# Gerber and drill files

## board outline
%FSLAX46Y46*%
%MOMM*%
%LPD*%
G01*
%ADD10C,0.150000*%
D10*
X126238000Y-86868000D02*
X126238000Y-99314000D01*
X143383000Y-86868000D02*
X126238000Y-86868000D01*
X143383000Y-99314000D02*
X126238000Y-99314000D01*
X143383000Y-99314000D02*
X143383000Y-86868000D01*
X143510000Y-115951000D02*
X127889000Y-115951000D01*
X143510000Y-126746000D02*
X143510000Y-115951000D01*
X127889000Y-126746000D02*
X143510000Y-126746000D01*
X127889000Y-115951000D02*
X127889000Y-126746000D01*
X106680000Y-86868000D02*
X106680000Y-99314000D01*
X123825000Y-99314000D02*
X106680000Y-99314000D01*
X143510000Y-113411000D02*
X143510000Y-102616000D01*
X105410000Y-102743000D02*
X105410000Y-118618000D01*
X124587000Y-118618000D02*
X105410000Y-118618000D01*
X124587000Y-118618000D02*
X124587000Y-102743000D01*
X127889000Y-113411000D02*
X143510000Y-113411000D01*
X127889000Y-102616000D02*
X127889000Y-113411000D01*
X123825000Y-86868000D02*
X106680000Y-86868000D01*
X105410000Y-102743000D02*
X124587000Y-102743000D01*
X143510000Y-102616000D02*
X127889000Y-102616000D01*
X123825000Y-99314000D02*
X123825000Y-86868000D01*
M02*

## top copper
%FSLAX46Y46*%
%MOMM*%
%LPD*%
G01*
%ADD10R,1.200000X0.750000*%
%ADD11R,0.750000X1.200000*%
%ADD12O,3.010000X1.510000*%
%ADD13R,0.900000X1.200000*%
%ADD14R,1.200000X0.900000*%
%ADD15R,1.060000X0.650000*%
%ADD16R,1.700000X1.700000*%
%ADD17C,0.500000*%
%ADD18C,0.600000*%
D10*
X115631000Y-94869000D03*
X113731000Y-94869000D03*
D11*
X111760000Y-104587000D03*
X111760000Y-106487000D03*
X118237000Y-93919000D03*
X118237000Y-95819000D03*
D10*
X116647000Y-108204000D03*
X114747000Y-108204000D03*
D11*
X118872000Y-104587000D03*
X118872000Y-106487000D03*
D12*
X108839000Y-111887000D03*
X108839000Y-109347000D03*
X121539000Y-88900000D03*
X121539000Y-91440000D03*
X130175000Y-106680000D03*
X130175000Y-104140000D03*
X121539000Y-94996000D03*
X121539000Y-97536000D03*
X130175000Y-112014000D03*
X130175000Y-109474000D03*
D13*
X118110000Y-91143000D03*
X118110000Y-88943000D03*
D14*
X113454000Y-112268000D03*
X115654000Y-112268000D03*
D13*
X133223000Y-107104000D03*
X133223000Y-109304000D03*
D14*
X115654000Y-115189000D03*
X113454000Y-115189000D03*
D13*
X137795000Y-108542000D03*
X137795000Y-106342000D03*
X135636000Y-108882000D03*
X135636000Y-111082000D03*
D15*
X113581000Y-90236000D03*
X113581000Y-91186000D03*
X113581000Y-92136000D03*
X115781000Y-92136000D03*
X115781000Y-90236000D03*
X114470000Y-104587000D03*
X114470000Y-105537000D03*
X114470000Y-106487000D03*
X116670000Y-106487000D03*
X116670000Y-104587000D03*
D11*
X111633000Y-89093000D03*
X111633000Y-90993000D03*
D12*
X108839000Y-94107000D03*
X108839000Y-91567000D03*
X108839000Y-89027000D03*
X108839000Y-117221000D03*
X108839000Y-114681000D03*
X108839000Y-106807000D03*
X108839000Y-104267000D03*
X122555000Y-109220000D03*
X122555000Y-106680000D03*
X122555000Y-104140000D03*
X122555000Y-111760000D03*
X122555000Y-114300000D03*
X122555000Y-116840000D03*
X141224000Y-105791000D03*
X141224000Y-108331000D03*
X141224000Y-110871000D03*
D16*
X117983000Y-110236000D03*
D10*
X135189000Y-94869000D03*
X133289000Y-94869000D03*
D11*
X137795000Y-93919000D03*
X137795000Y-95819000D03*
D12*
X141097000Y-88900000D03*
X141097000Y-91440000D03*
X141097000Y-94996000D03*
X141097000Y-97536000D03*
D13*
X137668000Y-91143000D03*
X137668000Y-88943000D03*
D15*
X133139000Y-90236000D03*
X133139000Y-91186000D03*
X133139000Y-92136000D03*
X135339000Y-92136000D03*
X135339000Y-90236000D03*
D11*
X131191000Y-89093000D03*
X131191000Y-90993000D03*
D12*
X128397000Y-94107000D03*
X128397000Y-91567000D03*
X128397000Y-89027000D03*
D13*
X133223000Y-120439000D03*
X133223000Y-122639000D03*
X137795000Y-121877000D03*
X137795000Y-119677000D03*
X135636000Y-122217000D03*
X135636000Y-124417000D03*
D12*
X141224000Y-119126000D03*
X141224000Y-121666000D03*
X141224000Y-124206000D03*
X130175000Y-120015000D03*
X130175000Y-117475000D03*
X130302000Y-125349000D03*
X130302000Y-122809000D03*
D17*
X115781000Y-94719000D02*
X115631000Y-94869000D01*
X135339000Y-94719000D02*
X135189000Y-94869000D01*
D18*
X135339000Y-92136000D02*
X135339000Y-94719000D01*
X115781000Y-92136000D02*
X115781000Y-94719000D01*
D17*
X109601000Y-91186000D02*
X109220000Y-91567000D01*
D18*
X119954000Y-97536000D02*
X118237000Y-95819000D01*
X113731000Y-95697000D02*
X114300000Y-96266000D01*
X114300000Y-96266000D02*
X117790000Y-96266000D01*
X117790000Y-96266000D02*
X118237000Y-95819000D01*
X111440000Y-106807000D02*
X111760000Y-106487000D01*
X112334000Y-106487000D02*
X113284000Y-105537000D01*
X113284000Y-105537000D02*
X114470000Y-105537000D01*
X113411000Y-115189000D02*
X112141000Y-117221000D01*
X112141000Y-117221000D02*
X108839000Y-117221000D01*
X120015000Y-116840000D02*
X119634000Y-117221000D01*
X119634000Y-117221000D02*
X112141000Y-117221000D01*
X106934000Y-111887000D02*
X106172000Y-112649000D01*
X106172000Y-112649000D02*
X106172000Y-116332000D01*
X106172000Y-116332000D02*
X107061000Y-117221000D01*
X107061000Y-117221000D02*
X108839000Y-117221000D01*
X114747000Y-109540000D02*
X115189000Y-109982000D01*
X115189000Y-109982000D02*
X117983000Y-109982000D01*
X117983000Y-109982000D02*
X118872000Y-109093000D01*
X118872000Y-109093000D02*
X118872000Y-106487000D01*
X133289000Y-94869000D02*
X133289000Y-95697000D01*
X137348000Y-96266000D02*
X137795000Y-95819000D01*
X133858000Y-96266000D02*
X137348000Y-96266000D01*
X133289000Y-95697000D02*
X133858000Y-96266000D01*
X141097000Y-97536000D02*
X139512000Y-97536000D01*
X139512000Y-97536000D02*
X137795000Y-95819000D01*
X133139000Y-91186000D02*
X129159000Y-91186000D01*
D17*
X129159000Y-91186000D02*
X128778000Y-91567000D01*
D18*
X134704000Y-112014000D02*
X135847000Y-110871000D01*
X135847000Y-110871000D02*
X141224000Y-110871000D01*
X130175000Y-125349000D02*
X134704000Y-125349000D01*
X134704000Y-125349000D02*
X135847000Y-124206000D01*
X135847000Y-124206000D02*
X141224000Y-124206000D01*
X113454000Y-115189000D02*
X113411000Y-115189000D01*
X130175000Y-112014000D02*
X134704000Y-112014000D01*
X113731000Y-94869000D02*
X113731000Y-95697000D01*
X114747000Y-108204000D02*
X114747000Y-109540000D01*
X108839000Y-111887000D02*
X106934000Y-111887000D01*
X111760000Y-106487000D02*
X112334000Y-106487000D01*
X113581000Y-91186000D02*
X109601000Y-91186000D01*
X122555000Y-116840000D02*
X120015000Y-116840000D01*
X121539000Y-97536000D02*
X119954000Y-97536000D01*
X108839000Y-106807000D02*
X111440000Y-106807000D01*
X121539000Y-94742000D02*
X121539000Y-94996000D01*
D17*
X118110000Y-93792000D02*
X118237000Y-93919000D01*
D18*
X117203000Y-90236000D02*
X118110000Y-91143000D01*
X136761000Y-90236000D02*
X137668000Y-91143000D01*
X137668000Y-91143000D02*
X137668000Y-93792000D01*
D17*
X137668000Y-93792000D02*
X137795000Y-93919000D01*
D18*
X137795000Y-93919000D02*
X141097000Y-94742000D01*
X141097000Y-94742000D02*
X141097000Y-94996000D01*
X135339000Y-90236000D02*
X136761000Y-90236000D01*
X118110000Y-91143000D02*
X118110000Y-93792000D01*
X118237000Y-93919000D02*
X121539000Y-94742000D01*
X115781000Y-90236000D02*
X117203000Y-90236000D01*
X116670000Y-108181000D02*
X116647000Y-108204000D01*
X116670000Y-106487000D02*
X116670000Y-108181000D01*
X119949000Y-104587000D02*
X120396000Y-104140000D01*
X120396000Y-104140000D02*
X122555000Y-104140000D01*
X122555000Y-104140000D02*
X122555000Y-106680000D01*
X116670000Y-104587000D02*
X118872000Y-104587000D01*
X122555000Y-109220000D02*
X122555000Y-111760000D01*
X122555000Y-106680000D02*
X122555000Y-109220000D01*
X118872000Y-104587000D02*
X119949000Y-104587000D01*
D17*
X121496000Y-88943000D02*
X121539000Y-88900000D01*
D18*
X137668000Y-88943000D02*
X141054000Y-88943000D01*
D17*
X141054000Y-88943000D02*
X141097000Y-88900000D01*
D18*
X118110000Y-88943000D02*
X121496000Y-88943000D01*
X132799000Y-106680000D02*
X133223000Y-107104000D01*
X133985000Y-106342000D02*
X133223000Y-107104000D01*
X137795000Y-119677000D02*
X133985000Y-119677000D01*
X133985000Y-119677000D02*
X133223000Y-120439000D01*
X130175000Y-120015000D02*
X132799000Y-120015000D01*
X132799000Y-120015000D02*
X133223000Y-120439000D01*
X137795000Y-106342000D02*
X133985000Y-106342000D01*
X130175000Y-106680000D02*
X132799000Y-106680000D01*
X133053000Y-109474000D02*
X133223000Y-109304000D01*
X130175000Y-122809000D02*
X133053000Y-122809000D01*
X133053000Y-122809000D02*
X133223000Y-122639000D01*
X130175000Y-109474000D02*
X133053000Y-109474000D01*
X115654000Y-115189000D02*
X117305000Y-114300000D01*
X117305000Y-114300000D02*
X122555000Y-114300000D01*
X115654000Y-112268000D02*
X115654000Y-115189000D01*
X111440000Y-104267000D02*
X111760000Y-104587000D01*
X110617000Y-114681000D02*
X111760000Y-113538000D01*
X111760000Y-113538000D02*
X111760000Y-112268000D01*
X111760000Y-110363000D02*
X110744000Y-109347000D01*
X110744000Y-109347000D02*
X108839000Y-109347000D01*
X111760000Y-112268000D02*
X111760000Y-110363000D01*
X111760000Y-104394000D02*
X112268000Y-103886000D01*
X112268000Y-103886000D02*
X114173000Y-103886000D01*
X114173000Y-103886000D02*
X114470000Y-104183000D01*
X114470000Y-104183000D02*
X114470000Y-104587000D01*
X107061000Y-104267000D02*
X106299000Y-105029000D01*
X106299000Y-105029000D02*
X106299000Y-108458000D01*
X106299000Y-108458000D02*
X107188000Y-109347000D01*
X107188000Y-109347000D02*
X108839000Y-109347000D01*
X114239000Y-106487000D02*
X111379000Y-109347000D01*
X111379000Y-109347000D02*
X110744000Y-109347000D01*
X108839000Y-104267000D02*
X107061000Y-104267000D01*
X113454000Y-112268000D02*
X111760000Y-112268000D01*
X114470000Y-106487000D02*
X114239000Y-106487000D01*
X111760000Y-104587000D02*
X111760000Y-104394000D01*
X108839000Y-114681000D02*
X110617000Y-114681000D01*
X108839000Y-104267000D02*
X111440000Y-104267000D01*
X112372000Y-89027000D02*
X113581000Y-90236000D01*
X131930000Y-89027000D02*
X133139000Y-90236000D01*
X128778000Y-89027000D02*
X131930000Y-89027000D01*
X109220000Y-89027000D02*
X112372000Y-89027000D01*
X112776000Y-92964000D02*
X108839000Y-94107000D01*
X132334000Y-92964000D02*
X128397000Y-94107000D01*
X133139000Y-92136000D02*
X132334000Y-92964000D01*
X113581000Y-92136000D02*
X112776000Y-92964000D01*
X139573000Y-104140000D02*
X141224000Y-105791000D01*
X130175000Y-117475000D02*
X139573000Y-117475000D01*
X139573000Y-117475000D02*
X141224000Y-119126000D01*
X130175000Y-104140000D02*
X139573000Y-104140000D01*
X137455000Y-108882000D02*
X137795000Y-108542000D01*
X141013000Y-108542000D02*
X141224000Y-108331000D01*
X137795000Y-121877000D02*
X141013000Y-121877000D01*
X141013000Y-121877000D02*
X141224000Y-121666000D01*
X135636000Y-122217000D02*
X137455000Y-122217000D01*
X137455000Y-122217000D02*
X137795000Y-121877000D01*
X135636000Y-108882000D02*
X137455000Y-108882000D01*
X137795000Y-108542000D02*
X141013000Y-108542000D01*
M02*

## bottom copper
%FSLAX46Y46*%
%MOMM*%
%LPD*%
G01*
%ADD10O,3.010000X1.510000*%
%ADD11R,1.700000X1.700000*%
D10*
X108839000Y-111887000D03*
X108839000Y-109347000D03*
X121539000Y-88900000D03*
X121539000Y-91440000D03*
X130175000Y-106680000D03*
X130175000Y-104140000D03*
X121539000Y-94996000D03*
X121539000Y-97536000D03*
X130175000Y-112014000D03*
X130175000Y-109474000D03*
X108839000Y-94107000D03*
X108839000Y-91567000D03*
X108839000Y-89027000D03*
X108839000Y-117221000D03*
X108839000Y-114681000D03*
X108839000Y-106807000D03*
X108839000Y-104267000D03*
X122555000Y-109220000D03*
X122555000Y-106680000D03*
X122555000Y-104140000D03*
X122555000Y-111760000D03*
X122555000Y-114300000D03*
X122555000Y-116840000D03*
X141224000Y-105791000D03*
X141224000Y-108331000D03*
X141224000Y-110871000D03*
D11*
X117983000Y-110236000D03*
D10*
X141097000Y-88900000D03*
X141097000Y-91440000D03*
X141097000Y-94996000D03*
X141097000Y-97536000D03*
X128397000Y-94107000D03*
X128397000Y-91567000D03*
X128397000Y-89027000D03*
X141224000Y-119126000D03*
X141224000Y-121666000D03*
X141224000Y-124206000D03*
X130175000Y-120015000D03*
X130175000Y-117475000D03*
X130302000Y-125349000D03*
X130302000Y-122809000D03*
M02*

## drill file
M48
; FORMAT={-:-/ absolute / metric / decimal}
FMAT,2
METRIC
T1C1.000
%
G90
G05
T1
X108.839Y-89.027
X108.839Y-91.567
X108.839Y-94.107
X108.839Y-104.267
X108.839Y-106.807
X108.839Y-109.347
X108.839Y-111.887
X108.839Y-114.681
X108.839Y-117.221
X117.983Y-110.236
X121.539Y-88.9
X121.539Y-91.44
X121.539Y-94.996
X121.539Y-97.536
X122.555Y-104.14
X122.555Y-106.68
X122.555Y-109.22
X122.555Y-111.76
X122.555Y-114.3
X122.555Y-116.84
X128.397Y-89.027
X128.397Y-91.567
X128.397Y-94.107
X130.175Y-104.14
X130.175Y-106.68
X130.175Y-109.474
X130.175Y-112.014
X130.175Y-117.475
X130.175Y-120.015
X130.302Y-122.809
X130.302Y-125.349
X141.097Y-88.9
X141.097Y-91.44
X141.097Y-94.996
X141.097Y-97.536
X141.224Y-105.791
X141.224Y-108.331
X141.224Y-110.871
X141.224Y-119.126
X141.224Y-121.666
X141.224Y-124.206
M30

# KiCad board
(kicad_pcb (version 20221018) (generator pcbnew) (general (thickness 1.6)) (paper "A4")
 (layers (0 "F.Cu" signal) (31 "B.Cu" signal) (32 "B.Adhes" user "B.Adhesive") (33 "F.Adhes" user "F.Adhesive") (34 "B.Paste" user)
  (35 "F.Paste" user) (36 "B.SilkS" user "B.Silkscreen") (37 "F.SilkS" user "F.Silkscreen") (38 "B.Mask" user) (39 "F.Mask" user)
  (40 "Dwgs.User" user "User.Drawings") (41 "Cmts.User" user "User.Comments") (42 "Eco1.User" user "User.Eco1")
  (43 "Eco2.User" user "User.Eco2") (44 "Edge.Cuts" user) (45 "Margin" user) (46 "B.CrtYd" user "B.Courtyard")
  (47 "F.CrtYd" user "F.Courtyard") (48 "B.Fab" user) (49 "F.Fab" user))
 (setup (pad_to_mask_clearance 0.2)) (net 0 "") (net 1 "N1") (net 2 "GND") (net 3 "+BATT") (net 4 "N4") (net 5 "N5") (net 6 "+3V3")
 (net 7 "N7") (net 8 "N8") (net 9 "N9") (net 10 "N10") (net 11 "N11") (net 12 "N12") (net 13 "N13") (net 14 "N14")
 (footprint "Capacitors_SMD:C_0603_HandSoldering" (layer "F.Cu") (at 114.681 94.869 180)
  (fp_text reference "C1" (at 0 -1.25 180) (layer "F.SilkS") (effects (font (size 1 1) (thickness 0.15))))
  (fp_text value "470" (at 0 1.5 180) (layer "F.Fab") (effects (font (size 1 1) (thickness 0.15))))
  (pad "1" smd rect (at -0.95 0 180) (size 1.2 0.75) (layers "F.Cu" "F.Paste" "F.Mask") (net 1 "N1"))
  (pad "2" smd rect (at 0.95 0 180) (size 1.2 0.75) (layers "F.Cu" "F.Paste" "F.Mask") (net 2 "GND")))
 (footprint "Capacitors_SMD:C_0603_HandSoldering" (layer "F.Cu") (at 111.76 105.537 -90)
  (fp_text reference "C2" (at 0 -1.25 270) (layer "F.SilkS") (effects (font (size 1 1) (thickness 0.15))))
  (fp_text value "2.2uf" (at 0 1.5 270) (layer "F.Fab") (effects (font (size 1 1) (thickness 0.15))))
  (pad "1" smd rect (at -0.95 0 270) (size 1.2 0.75) (layers "F.Cu" "F.Paste" "F.Mask") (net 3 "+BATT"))
  (pad "2" smd rect (at 0.95 0 270) (size 1.2 0.75) (layers "F.Cu" "F.Paste" "F.Mask") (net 2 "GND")))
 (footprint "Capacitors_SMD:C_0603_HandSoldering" (layer "F.Cu") (at 118.237 94.869 -90)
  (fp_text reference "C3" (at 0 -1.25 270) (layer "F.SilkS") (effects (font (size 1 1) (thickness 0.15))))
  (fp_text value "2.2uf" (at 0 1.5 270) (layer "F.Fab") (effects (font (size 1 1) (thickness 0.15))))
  (pad "1" smd rect (at -0.95 0 270) (size 1.2 0.75) (layers "F.Cu" "F.Paste" "F.Mask") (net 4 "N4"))
  (pad "2" smd rect (at 0.95 0 270) (size 1.2 0.75) (layers "F.Cu" "F.Paste" "F.Mask") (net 2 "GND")))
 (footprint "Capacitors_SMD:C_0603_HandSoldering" (layer "F.Cu") (at 115.697 108.204 180)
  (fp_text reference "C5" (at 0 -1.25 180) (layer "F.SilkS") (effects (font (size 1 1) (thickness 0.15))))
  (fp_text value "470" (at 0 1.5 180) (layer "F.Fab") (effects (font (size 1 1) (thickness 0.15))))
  (pad "1" smd rect (at -0.95 0 180) (size 1.2 0.75) (layers "F.Cu" "F.Paste" "F.Mask") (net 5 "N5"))
  (pad "2" smd rect (at 0.95 0 180) (size 1.2 0.75) (layers "F.Cu" "F.Paste" "F.Mask") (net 2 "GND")))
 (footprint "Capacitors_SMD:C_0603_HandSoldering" (layer "F.Cu") (at 118.872 105.537 -90)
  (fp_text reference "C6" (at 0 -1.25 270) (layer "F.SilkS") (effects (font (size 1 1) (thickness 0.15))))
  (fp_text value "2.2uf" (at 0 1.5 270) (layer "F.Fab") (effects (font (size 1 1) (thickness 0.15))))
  (pad "1" smd rect (at -0.95 0 270) (size 1.2 0.75) (layers "F.Cu" "F.Paste" "F.Mask") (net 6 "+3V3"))
  (pad "2" smd rect (at 0.95 0 270) (size 1.2 0.75) (layers "F.Cu" "F.Paste" "F.Mask") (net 2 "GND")))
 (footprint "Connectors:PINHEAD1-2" (layer "F.Cu") (at 108.839 111.887 90)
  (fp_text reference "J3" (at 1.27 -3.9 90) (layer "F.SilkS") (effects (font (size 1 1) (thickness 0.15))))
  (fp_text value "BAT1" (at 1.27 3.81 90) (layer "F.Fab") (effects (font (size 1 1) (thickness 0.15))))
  (pad "1" thru_hole oval (at 0 0 90) (size 1.51 3.01) (drill 1) (layers "*.Cu" "*.Mask") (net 2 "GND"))
  (pad "2" thru_hole oval (at 2.54 0 90) (size 1.51 3.01) (drill 1) (layers "*.Cu" "*.Mask") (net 3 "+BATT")))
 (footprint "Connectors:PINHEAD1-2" (layer "F.Cu") (at 121.539 88.9 -90)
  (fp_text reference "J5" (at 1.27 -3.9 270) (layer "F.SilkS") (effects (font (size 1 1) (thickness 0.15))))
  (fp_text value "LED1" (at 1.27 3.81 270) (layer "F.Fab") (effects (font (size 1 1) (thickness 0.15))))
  (pad "1" thru_hole oval (at 0 0 270) (size 1.51 3.01) (drill 1) (layers "*.Cu" "*.Mask") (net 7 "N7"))
  (pad "2" thru_hole oval (at 2.54 0 270) (size 1.51 3.01) (drill 1) (layers "*.Cu" "*.Mask") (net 2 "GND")))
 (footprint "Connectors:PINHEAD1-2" (layer "F.Cu") (at 130.175 106.68 90)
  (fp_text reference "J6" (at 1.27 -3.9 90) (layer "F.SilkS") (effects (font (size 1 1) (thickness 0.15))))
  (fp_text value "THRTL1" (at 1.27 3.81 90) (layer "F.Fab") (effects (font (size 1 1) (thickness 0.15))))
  (pad "1" thru_hole oval (at 0 0 90) (size 1.51 3.01) (drill 1) (layers "*.Cu" "*.Mask") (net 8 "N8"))
  (pad "2" thru_hole oval (at 2.54 0 90) (size 1.51 3.01) (drill 1) (layers "*.Cu" "*.Mask") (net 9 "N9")))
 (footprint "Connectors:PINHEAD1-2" (layer "F.Cu") (at 121.539 94.996 -90)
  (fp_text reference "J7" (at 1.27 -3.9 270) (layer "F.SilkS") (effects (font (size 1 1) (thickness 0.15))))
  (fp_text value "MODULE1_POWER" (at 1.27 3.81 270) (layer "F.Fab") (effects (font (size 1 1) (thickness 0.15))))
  (pad "1" thru_hole oval (at 0 0 270) (size 1.51 3.01) (drill 1) (layers "*.Cu" "*.Mask") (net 4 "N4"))
  (pad "2" thru_hole oval (at 2.54 0 270) (size 1.51 3.01) (drill 1) (layers "*.Cu" "*.Mask") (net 2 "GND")))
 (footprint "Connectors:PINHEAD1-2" (layer "F.Cu") (at 130.175 112.014 90)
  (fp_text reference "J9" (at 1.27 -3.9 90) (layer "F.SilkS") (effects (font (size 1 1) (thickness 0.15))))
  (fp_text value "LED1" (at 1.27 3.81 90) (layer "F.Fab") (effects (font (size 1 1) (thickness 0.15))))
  (pad "1" thru_hole oval (at 0 0 90) (size 1.51 3.01) (drill 1) (layers "*.Cu" "*.Mask") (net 2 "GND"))
  (pad "2" thru_hole oval (at 2.54 0 90) (size 1.51 3.01) (drill 1) (layers "*.Cu" "*.Mask") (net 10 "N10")))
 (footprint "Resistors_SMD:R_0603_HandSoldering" (layer "F.Cu") (at 118.11 90.043 90)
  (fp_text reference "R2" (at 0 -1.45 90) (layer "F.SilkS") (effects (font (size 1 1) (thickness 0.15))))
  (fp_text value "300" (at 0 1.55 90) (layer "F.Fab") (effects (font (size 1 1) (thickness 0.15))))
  (pad "1" smd rect (at -1.1 0 90) (size 1.2 0.9) (layers "F.Cu" "F.Paste" "F.Mask") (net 4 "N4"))
  (pad "2" smd rect (at 1.1 0 90) (size 1.2 0.9) (layers "F.Cu" "F.Paste" "F.Mask") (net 7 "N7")))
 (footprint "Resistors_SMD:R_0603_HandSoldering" (layer "F.Cu") (at 114.554 112.268)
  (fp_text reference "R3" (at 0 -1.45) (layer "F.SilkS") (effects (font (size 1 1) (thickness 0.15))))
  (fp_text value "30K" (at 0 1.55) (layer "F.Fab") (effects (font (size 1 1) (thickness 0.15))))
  (pad "1" smd rect (at -1.1 0) (size 1.2 0.9) (layers "F.Cu" "F.Paste" "F.Mask") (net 3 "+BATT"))
  (pad "2" smd rect (at 1.1 0) (size 1.2 0.9) (layers "F.Cu" "F.Paste" "F.Mask") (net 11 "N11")))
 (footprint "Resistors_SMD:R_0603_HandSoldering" (layer "F.Cu") (at 133.223 108.204 -90)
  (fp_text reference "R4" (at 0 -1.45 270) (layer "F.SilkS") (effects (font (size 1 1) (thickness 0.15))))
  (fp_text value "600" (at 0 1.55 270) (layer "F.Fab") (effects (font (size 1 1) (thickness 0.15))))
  (pad "1" smd rect (at -1.1 0 270) (size 1.2 0.9) (layers "F.Cu" "F.Paste" "F.Mask") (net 8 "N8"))
  (pad "2" smd rect (at 1.1 0 270) (size 1.2 0.9) (layers "F.Cu" "F.Paste" "F.Mask") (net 10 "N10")))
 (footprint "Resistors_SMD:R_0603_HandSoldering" (layer "F.Cu") (at 114.554 115.189 180)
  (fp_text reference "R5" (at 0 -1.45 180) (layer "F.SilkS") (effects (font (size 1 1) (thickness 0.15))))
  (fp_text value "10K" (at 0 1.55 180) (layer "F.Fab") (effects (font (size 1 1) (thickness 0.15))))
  (pad "1" smd rect (at -1.1 0 180) (size 1.2 0.9) (layers "F.Cu" "F.Paste" "F.Mask") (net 11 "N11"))
  (pad "2" smd rect (at 1.1 0 180) (size 1.2 0.9) (layers "F.Cu" "F.Paste" "F.Mask") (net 2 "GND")))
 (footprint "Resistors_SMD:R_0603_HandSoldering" (layer "F.Cu") (at 137.795 107.442 90)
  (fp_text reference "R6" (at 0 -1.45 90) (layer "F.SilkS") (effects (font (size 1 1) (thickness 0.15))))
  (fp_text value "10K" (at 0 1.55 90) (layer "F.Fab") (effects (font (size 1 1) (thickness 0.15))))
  (pad "1" smd rect (at -1.1 0 90) (size 1.2 0.9) (layers "F.Cu" "F.Paste" "F.Mask") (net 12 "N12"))
  (pad "2" smd rect (at 1.1 0 90) (size 1.2 0.9) (layers "F.Cu" "F.Paste" "F.Mask") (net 8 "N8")))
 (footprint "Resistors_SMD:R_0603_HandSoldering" (layer "F.Cu") (at 135.636 109.982 -90)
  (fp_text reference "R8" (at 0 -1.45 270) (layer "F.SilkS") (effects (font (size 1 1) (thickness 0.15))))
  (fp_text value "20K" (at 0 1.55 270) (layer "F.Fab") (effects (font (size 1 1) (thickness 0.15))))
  (pad "1" smd rect (at -1.1 0 270) (size 1.2 0.9) (layers "F.Cu" "F.Paste" "F.Mask") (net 12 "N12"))
  (pad "2" smd rect (at 1.1 0 270) (size 1.2 0.9) (layers "F.Cu" "F.Paste" "F.Mask") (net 2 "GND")))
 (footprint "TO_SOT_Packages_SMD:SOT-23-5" (layer "F.Cu") (at 114.681 91.186)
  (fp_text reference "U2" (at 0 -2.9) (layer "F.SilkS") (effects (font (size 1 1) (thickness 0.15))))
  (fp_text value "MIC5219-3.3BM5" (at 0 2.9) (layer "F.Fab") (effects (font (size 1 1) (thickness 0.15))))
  (pad "1" smd rect (at -1.1 -0.95) (size 1.06 0.65) (layers "F.Cu" "F.Paste" "F.Mask") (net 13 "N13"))
  (pad "2" smd rect (at -1.1 0) (size 1.06 0.65) (layers "F.Cu" "F.Paste" "F.Mask") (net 2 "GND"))
  (pad "3" smd rect (at -1.1 0.95) (size 1.06 0.65) (layers "F.Cu" "F.Paste" "F.Mask") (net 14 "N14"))
  (pad "4" smd rect (at 1.1 0.95) (size 1.06 0.65) (layers "F.Cu" "F.Paste" "F.Mask") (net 1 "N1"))
  (pad "5" smd rect (at 1.1 -0.95) (size 1.06 0.65) (layers "F.Cu" "F.Paste" "F.Mask") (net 4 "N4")))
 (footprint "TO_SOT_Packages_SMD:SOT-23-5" (layer "F.Cu") (at 115.57 105.537)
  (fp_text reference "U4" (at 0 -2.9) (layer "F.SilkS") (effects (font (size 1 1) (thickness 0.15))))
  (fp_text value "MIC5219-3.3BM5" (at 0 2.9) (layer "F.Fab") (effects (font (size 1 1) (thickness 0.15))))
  (pad "1" smd rect (at -1.1 -0.95) (size 1.06 0.65) (layers "F.Cu" "F.Paste" "F.Mask") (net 3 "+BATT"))
  (pad "2" smd rect (at -1.1 0) (size 1.06 0.65) (layers "F.Cu" "F.Paste" "F.Mask") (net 2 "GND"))
  (pad "3" smd rect (at -1.1 0.95) (size 1.06 0.65) (layers "F.Cu" "F.Paste" "F.Mask") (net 3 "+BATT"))
  (pad "4" smd rect (at 1.1 0.95) (size 1.06 0.65) (layers "F.Cu" "F.Paste" "F.Mask") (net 5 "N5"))
  (pad "5" smd rect (at 1.1 -0.95) (size 1.06 0.65) (layers "F.Cu" "F.Paste" "F.Mask") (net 6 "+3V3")))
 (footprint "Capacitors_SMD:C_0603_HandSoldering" (layer "F.Cu") (at 111.633 90.043 -90)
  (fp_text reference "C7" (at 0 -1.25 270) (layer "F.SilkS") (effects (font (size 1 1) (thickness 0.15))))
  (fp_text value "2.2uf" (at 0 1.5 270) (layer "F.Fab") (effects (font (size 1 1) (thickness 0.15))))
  (pad "1" smd rect (at -0.95 0 270) (size 1.2 0.75) (layers "F.Cu" "F.Paste" "F.Mask") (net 13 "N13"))
  (pad "2" smd rect (at 0.95 0 270) (size 1.2 0.75) (layers "F.Cu" "F.Paste" "F.Mask") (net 2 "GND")))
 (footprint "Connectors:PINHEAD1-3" (layer "F.Cu") (at 108.839 94.107 90)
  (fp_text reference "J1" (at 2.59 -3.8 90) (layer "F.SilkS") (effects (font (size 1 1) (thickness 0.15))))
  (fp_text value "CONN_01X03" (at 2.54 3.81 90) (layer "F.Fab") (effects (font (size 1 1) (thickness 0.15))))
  (pad "1" thru_hole oval (at 0 0 90) (size 1.51 3.01) (drill 1) (layers "*.Cu" "*.Mask") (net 14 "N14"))
  (pad "2" thru_hole oval (at 2.54 0 90) (size 1.51 3.01) (drill 1) (layers "*.Cu" "*.Mask") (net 2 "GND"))
  (pad "3" thru_hole oval (at 5.08 0 90) (size 1.51 3.01) (drill 1) (layers "*.Cu" "*.Mask") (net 13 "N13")))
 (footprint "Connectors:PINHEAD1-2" (layer "F.Cu") (at 108.839 117.221 90)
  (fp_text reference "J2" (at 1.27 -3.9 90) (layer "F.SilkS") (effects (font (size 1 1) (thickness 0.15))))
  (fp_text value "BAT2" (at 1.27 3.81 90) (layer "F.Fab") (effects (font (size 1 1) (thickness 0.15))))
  (pad "1" thru_hole oval (at 0 0 90) (size 1.51 3.01) (drill 1) (layers "*.Cu" "*.Mask") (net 2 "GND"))
  (pad "2" thru_hole oval (at 2.54 0 90) (size 1.51 3.01) (drill 1) (layers "*.Cu" "*.Mask") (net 3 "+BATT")))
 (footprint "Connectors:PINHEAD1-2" (layer "F.Cu") (at 108.839 106.807 90)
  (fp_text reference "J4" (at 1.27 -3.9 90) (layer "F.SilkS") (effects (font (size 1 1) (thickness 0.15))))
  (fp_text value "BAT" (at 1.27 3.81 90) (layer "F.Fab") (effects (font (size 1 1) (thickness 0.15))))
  (pad "1" thru_hole oval (at 0 0 90) (size 1.51 3.01) (drill 1) (layers "*.Cu" "*.Mask") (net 2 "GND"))
  (pad "2" thru_hole oval (at 2.54 0 90) (size 1.51 3.01) (drill 1) (layers "*.Cu" "*.Mask") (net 3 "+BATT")))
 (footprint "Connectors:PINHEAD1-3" (layer "F.Cu") (at 122.555 109.22 90)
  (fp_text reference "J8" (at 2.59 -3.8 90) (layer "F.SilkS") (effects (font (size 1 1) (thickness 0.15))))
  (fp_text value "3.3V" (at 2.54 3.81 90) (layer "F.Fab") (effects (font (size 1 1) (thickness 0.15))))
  (pad "1" thru_hole oval (at 0 0 90) (size 1.51 3.01) (drill 1) (layers "*.Cu" "*.Mask") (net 6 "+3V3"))
  (pad "2" thru_hole oval (at 2.54 0 90) (size 1.51 3.01) (drill 1) (layers "*.Cu" "*.Mask") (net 6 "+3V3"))
  (pad "3" thru_hole oval (at 5.08 0 90) (size 1.51 3.01) (drill 1) (layers "*.Cu" "*.Mask") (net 6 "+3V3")))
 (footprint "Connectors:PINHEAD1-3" (layer "F.Cu") (at 122.555 111.76 -90)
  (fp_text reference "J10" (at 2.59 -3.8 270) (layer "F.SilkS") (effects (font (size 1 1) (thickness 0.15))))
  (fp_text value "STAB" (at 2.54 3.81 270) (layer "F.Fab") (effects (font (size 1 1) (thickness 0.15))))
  (pad "1" thru_hole oval (at 0 0 270) (size 1.51 3.01) (drill 1) (layers "*.Cu" "*.Mask") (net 6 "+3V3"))
  (pad "2" thru_hole oval (at 2.54 0 270) (size 1.51 3.01) (drill 1) (layers "*.Cu" "*.Mask") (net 11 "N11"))
  (pad "3" thru_hole oval (at 5.08 0 270) (size 1.51 3.01) (drill 1) (layers "*.Cu" "*.Mask") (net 2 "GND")))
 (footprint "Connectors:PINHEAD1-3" (layer "F.Cu") (at 141.224 105.791 -90)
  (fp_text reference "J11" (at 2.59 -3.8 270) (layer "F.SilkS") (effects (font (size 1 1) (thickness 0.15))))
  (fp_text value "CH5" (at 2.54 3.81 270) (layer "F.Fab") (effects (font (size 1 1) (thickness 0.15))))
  (pad "1" thru_hole oval (at 0 0 270) (size 1.51 3.01) (drill 1) (layers "*.Cu" "*.Mask") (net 9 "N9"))
  (pad "2" thru_hole oval (at 2.54 0 270) (size 1.51 3.01) (drill 1) (layers "*.Cu" "*.Mask") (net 12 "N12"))
  (pad "3" thru_hole oval (at 5.08 0 270) (size 1.51 3.01) (drill 1) (layers "*.Cu" "*.Mask") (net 2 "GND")))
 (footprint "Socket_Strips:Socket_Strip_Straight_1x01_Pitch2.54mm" (layer "F.Cu") (at 117.983 110.236)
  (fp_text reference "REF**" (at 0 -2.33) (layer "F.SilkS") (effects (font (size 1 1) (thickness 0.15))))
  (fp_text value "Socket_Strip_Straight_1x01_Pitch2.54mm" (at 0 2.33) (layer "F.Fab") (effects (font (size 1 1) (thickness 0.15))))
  (pad "1" thru_hole rect (at 0 0) (size 1.7 1.7) (drill 1) (layers "*.Cu" "*.Mask")))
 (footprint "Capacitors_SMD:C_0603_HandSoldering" (layer "F.Cu") (at 134.239 94.869 180)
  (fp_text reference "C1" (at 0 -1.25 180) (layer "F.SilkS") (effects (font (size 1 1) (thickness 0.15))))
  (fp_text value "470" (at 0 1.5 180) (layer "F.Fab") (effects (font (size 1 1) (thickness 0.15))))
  (pad "1" smd rect (at -0.95 0 180) (size 1.2 0.75) (layers "F.Cu" "F.Paste" "F.Mask") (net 1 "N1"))
  (pad "2" smd rect (at 0.95 0 180) (size 1.2 0.75) (layers "F.Cu" "F.Paste" "F.Mask") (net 2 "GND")))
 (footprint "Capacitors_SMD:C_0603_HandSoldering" (layer "F.Cu") (at 137.795 94.869 -90)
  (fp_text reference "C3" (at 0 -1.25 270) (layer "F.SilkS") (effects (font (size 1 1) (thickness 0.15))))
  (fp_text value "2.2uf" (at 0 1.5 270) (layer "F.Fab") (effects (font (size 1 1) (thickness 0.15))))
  (pad "1" smd rect (at -0.95 0 270) (size 1.2 0.75) (layers "F.Cu" "F.Paste" "F.Mask") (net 4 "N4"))
  (pad "2" smd rect (at 0.95 0 270) (size 1.2 0.75) (layers "F.Cu" "F.Paste" "F.Mask") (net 2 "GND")))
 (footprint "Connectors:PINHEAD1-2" (layer "F.Cu") (at 141.097 88.9 -90)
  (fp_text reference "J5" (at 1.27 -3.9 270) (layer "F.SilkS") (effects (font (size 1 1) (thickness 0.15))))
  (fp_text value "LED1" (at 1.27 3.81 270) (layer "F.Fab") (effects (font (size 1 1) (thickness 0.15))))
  (pad "1" thru_hole oval (at 0 0 270) (size 1.51 3.01) (drill 1) (layers "*.Cu" "*.Mask") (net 7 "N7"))
  (pad "2" thru_hole oval (at 2.54 0 270) (size 1.51 3.01) (drill 1) (layers "*.Cu" "*.Mask") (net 2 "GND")))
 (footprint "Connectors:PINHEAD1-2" (layer "F.Cu") (at 141.097 94.996 -90)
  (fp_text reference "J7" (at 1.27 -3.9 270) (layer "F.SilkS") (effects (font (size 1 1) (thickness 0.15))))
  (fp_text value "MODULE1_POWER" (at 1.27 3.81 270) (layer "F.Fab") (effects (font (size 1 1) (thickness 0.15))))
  (pad "1" thru_hole oval (at 0 0 270) (size 1.51 3.01) (drill 1) (layers "*.Cu" "*.Mask") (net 4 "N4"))
  (pad "2" thru_hole oval (at 2.54 0 270) (size 1.51 3.01) (drill 1) (layers "*.Cu" "*.Mask") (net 2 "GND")))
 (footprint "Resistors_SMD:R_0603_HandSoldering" (layer "F.Cu") (at 137.668 90.043 90)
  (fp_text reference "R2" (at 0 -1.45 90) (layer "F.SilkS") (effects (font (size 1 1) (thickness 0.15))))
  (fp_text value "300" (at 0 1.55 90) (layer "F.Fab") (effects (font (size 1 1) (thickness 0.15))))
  (pad "1" smd rect (at -1.1 0 90) (size 1.2 0.9) (layers "F.Cu" "F.Paste" "F.Mask") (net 4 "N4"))
  (pad "2" smd rect (at 1.1 0 90) (size 1.2 0.9) (layers "F.Cu" "F.Paste" "F.Mask") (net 7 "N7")))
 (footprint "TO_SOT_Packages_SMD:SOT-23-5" (layer "F.Cu") (at 134.239 91.186)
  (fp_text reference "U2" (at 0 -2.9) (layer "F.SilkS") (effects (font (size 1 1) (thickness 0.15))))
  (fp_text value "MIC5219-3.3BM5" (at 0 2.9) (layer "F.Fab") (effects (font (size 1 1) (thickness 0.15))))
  (pad "1" smd rect (at -1.1 -0.95) (size 1.06 0.65) (layers "F.Cu" "F.Paste" "F.Mask") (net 13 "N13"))
  (pad "2" smd rect (at -1.1 0) (size 1.06 0.65) (layers "F.Cu" "F.Paste" "F.Mask") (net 2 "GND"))
  (pad "3" smd rect (at -1.1 0.95) (size 1.06 0.65) (layers "F.Cu" "F.Paste" "F.Mask") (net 14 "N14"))
  (pad "4" smd rect (at 1.1 0.95) (size 1.06 0.65) (layers "F.Cu" "F.Paste" "F.Mask") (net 1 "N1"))
  (pad "5" smd rect (at 1.1 -0.95) (size 1.06 0.65) (layers "F.Cu" "F.Paste" "F.Mask") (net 4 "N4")))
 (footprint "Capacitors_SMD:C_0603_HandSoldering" (layer "F.Cu") (at 131.191 90.043 -90)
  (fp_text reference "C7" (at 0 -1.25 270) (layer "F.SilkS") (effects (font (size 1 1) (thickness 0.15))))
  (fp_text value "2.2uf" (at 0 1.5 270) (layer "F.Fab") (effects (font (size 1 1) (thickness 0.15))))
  (pad "1" smd rect (at -0.95 0 270) (size 1.2 0.75) (layers "F.Cu" "F.Paste" "F.Mask") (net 13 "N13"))
  (pad "2" smd rect (at 0.95 0 270) (size 1.2 0.75) (layers "F.Cu" "F.Paste" "F.Mask") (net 2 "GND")))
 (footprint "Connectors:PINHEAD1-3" (layer "F.Cu") (at 128.397 94.107 90)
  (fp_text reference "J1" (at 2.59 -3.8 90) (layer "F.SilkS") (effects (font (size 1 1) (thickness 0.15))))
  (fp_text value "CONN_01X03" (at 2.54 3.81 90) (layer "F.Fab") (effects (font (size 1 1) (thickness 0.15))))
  (pad "1" thru_hole oval (at 0 0 90) (size 1.51 3.01) (drill 1) (layers "*.Cu" "*.Mask") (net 14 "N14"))
  (pad "2" thru_hole oval (at 2.54 0 90) (size 1.51 3.01) (drill 1) (layers "*.Cu" "*.Mask") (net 2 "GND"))
  (pad "3" thru_hole oval (at 5.08 0 90) (size 1.51 3.01) (drill 1) (layers "*.Cu" "*.Mask") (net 13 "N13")))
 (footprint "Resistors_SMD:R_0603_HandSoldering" (layer "F.Cu") (at 133.223 121.539 -90)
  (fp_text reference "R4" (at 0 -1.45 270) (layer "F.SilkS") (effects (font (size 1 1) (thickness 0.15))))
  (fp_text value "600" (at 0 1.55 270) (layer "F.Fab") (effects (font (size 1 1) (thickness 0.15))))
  (pad "1" smd rect (at -1.1 0 270) (size 1.2 0.9) (layers "F.Cu" "F.Paste" "F.Mask") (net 8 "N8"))
  (pad "2" smd rect (at 1.1 0 270) (size 1.2 0.9) (layers "F.Cu" "F.Paste" "F.Mask") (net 10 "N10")))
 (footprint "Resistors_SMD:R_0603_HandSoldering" (layer "F.Cu") (at 137.795 120.777 90)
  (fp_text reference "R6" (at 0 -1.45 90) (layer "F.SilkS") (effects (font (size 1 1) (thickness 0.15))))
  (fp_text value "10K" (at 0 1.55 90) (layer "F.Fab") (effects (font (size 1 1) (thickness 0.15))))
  (pad "1" smd rect (at -1.1 0 90) (size 1.2 0.9) (layers "F.Cu" "F.Paste" "F.Mask") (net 12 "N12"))
  (pad "2" smd rect (at 1.1 0 90) (size 1.2 0.9) (layers "F.Cu" "F.Paste" "F.Mask") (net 8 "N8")))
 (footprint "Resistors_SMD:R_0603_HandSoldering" (layer "F.Cu") (at 135.636 123.317 -90)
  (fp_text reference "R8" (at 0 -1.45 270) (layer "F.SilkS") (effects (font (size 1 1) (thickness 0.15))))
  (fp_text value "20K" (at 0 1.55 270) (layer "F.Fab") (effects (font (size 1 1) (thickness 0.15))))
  (pad "1" smd rect (at -1.1 0 270) (size 1.2 0.9) (layers "F.Cu" "F.Paste" "F.Mask") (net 12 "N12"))
  (pad "2" smd rect (at 1.1 0 270) (size 1.2 0.9) (layers "F.Cu" "F.Paste" "F.Mask") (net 2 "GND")))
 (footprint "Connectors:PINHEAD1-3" (layer "F.Cu") (at 141.224 119.126 -90)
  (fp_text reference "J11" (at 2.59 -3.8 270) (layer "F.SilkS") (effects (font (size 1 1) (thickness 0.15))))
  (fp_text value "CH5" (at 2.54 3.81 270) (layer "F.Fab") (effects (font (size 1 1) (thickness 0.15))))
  (pad "1" thru_hole oval (at 0 0 270) (size 1.51 3.01) (drill 1) (layers "*.Cu" "*.Mask") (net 9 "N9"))
  (pad "2" thru_hole oval (at 2.54 0 270) (size 1.51 3.01) (drill 1) (layers "*.Cu" "*.Mask") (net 12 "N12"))
  (pad "3" thru_hole oval (at 5.08 0 270) (size 1.51 3.01) (drill 1) (layers "*.Cu" "*.Mask") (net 2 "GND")))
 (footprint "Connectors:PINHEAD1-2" (layer "F.Cu") (at 130.175 120.015 90)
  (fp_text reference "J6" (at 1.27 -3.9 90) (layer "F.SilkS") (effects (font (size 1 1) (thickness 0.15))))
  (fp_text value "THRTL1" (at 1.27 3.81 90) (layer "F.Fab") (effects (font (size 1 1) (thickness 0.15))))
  (pad "1" thru_hole oval (at 0 0 90) (size 1.51 3.01) (drill 1) (layers "*.Cu" "*.Mask") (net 8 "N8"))
  (pad "2" thru_hole oval (at 2.54 0 90) (size 1.51 3.01) (drill 1) (layers "*.Cu" "*.Mask") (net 9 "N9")))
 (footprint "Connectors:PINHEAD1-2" (layer "F.Cu") (at 130.302 125.349 90)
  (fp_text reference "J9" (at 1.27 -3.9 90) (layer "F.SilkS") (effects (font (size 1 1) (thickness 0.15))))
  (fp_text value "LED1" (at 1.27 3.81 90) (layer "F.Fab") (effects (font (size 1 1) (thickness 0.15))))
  (pad "1" thru_hole oval (at 0 0 90) (size 1.51 3.01) (drill 1) (layers "*.Cu" "*.Mask") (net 2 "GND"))
  (pad "2" thru_hole oval (at 2.54 0 90) (size 1.51 3.01) (drill 1) (layers "*.Cu" "*.Mask") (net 10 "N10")))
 (gr_line (start 126.238 86.868) (end 126.238 99.314) (stroke (width 0.15) (type solid)) (layer "Edge.Cuts"))
 (gr_line (start 143.383 86.868) (end 126.238 86.868) (stroke (width 0.15) (type solid)) (layer "Edge.Cuts"))
 (gr_line (start 143.383 99.314) (end 126.238 99.314) (stroke (width 0.15) (type solid)) (layer "Edge.Cuts"))
 (gr_line (start 143.383 99.314) (end 143.383 86.868) (stroke (width 0.15) (type solid)) (layer "Edge.Cuts"))
 (gr_line (start 143.51 115.951) (end 127.889 115.951) (stroke (width 0.15) (type solid)) (layer "Edge.Cuts"))
 (gr_line (start 143.51 126.746) (end 143.51 115.951) (stroke (width 0.15) (type solid)) (layer "Edge.Cuts"))
 (gr_line (start 127.889 126.746) (end 143.51 126.746) (stroke (width 0.15) (type solid)) (layer "Edge.Cuts"))
 (gr_line (start 127.889 115.951) (end 127.889 126.746) (stroke (width 0.15) (type solid)) (layer "Edge.Cuts"))
 (gr_line (start 106.68 86.868) (end 106.68 99.314) (stroke (width 0.15) (type solid)) (layer "Edge.Cuts"))
 (gr_line (start 123.825 99.314) (end 106.68 99.314) (stroke (width 0.15) (type solid)) (layer "Edge.Cuts"))
 (gr_line (start 143.51 113.411) (end 143.51 102.616) (stroke (width 0.15) (type solid)) (layer "Edge.Cuts"))
 (gr_line (start 105.41 102.743) (end 105.41 118.618) (stroke (width 0.15) (type solid)) (layer "Edge.Cuts"))
 (gr_line (start 124.587 118.618) (end 105.41 118.618) (stroke (width 0.15) (type solid)) (layer "Edge.Cuts"))
 (gr_line (start 124.587 118.618) (end 124.587 102.743) (stroke (width 0.15) (type solid)) (layer "Edge.Cuts"))
 (gr_line (start 127.889 113.411) (end 143.51 113.411) (stroke (width 0.15) (type solid)) (layer "Edge.Cuts"))
 (gr_line (start 127.889 102.616) (end 127.889 113.411) (stroke (width 0.15) (type solid)) (layer "Edge.Cuts"))
 (gr_line (start 123.825 86.868) (end 106.68 86.868) (stroke (width 0.15) (type solid)) (layer "Edge.Cuts"))
 (gr_line (start 105.41 102.743) (end 124.587 102.743) (stroke (width 0.15) (type solid)) (layer "Edge.Cuts"))
 (gr_line (start 143.51 102.616) (end 127.889 102.616) (stroke (width 0.15) (type solid)) (layer "Edge.Cuts"))
 (gr_line (start 123.825 99.314) (end 123.825 86.868) (stroke (width 0.15) (type solid)) (layer "Edge.Cuts"))
 (segment (start 115.781 94.719) (end 115.631 94.869) (width 0.5) (layer "F.Cu") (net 1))
 (segment (start 135.339 94.719) (end 135.189 94.869) (width 0.5) (layer "F.Cu") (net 1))
 (segment (start 135.339 92.136) (end 135.339 94.719) (width 0.6) (layer "F.Cu") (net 1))
 (segment (start 115.781 92.136) (end 115.781 94.719) (width 0.6) (layer "F.Cu") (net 1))
 (segment (start 109.601 91.186) (end 109.22 91.567) (width 0.5) (layer "F.Cu") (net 2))
 (segment (start 119.954 97.536) (end 118.237 95.819) (width 0.6) (layer "F.Cu") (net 2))
 (segment (start 113.731 95.697) (end 114.3 96.266) (width 0.6) (layer "F.Cu") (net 2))
 (segment (start 114.3 96.266) (end 117.79 96.266) (width 0.6) (layer "F.Cu") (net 2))
 (segment (start 117.79 96.266) (end 118.237 95.819) (width 0.6) (layer "F.Cu") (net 2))
 (segment (start 111.44 106.807) (end 111.76 106.487) (width 0.6) (layer "F.Cu") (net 2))
 (segment (start 112.334 106.487) (end 113.284 105.537) (width 0.6) (layer "F.Cu") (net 2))
 (segment (start 113.284 105.537) (end 114.47 105.537) (width 0.6) (layer "F.Cu") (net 2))
 (segment (start 113.411 115.189) (end 112.141 117.221) (width 0.6) (layer "F.Cu") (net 2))
 (segment (start 112.141 117.221) (end 108.839 117.221) (width 0.6) (layer "F.Cu") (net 2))
 (segment (start 120.015 116.84) (end 119.634 117.221) (width 0.6) (layer "F.Cu") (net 2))
 (segment (start 119.634 117.221) (end 112.141 117.221) (width 0.6) (layer "F.Cu") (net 2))
 (segment (start 106.934 111.887) (end 106.172 112.649) (width 0.6) (layer "F.Cu") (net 2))
 (segment (start 106.172 112.649) (end 106.172 116.332) (width 0.6) (layer "F.Cu") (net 2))
 (segment (start 106.172 116.332) (end 107.061 117.221) (width 0.6) (layer "F.Cu") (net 2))
 (segment (start 107.061 117.221) (end 108.839 117.221) (width 0.6) (layer "F.Cu") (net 2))
 (segment (start 114.747 109.54) (end 115.189 109.982) (width 0.6) (layer "F.Cu") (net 2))
 (segment (start 115.189 109.982) (end 117.983 109.982) (width 0.6) (layer "F.Cu") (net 2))
 (segment (start 117.983 109.982) (end 118.872 109.093) (width 0.6) (layer "F.Cu") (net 2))
 (segment (start 118.872 109.093) (end 118.872 106.487) (width 0.6) (layer "F.Cu") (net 2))
 (segment (start 133.289 94.869) (end 133.289 95.697) (width 0.6) (layer "F.Cu") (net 2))
 (segment (start 137.348 96.266) (end 137.795 95.819) (width 0.6) (layer "F.Cu") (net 2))
 (segment (start 133.858 96.266) (end 137.348 96.266) (width 0.6) (layer "F.Cu") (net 2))
 (segment (start 133.289 95.697) (end 133.858 96.266) (width 0.6) (layer "F.Cu") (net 2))
 (segment (start 141.097 97.536) (end 139.512 97.536) (width 0.6) (layer "F.Cu") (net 2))
 (segment (start 139.512 97.536) (end 137.795 95.819) (width 0.6) (layer "F.Cu") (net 2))
 (segment (start 133.139 91.186) (end 129.159 91.186) (width 0.6) (layer "F.Cu") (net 2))
 (segment (start 129.159 91.186) (end 128.778 91.567) (width 0.5) (layer "F.Cu") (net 2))
 (segment (start 134.704 112.014) (end 135.847 110.871) (width 0.6) (layer "F.Cu") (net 2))
 (segment (start 135.847 110.871) (end 141.224 110.871) (width 0.6) (layer "F.Cu") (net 2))
 (segment (start 130.175 125.349) (end 134.704 125.349) (width 0.6) (layer "F.Cu") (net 2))
 (segment (start 134.704 125.349) (end 135.847 124.206) (width 0.6) (layer "F.Cu") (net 2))
 (segment (start 135.847 124.206) (end 141.224 124.206) (width 0.6) (layer "F.Cu") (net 2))
 (segment (start 113.454 115.189) (end 113.411 115.189) (width 0.6) (layer "F.Cu") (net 2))
 (segment (start 130.175 112.014) (end 134.704 112.014) (width 0.6) (layer "F.Cu") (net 2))
 (segment (start 113.731 94.869) (end 113.731 95.697) (width 0.6) (layer "F.Cu") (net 2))
 (segment (start 114.747 108.204) (end 114.747 109.54) (width 0.6) (layer "F.Cu") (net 2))
 (segment (start 108.839 111.887) (end 106.934 111.887) (width 0.6) (layer "F.Cu") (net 2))
 (segment (start 111.76 106.487) (end 112.334 106.487) (width 0.6) (layer "F.Cu") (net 2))
 (segment (start 113.581 91.186) (end 109.601 91.186) (width 0.6) (layer "F.Cu") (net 2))
 (segment (start 122.555 116.84) (end 120.015 116.84) (width 0.6) (layer "F.Cu") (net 2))
 (segment (start 121.539 97.536) (end 119.954 97.536) (width 0.6) (layer "F.Cu") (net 2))
 (segment (start 108.839 106.807) (end 111.44 106.807) (width 0.6) (layer "F.Cu") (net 2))
 (segment (start 121.539 94.742) (end 121.539 94.996) (width 0.6) (layer "F.Cu") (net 4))
 (segment (start 118.11 93.792) (end 118.237 93.919) (width 0.5) (layer "F.Cu") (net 4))
 (segment (start 117.203 90.236) (end 118.11 91.143) (width 0.6) (layer "F.Cu") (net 4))
 (segment (start 136.761 90.236) (end 137.668 91.143) (width 0.6) (layer "F.Cu") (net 4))
 (segment (start 137.668 91.143) (end 137.668 93.792) (width 0.6) (layer "F.Cu") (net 4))
 (segment (start 137.668 93.792) (end 137.795 93.919) (width 0.5) (layer "F.Cu") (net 4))
 (segment (start 137.795 93.919) (end 141.097 94.742) (width 0.6) (layer "F.Cu") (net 4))
 (segment (start 141.097 94.742) (end 141.097 94.996) (width 0.6) (layer "F.Cu") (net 4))
 (segment (start 135.339 90.236) (end 136.761 90.236) (width 0.6) (layer "F.Cu") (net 4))
 (segment (start 118.11 91.143) (end 118.11 93.792) (width 0.6) (layer "F.Cu") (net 4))
 (segment (start 118.237 93.919) (end 121.539 94.742) (width 0.6) (layer "F.Cu") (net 4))
 (segment (start 115.781 90.236) (end 117.203 90.236) (width 0.6) (layer "F.Cu") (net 4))
 (segment (start 116.67 108.181) (end 116.647 108.204) (width 0.6) (layer "F.Cu") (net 5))
 (segment (start 116.67 106.487) (end 116.67 108.181) (width 0.6) (layer "F.Cu") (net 5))
 (segment (start 119.949 104.587) (end 120.396 104.14) (width 0.6) (layer "F.Cu") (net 6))
 (segment (start 120.396 104.14) (end 122.555 104.14) (width 0.6) (layer "F.Cu") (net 6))
 (segment (start 122.555 104.14) (end 122.555 106.68) (width 0.6) (layer "F.Cu") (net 6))
 (segment (start 116.67 104.587) (end 118.872 104.587) (width 0.6) (layer "F.Cu") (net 6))
 (segment (start 122.555 109.22) (end 122.555 111.76) (width 0.6) (layer "F.Cu") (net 6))
 (segment (start 122.555 106.68) (end 122.555 109.22) (width 0.6) (layer "F.Cu") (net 6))
 (segment (start 118.872 104.587) (end 119.949 104.587) (width 0.6) (layer "F.Cu") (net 6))
 (segment (start 121.496 88.943) (end 121.539 88.9) (width 0.5) (layer "F.Cu") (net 7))
 (segment (start 137.668 88.943) (end 141.054 88.943) (width 0.6) (layer "F.Cu") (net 7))
 (segment (start 141.054 88.943) (end 141.097 88.9) (width 0.5) (layer "F.Cu") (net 7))
 (segment (start 118.11 88.943) (end 121.496 88.943) (width 0.6) (layer "F.Cu") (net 7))
 (segment (start 132.799 106.68) (end 133.223 107.104) (width 0.6) (layer "F.Cu") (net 8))
 (segment (start 133.985 106.342) (end 133.223 107.104) (width 0.6) (layer "F.Cu") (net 8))
 (segment (start 137.795 119.677) (end 133.985 119.677) (width 0.6) (layer "F.Cu") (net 8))
 (segment (start 133.985 119.677) (end 133.223 120.439) (width 0.6) (layer "F.Cu") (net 8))
 (segment (start 130.175 120.015) (end 132.799 120.015) (width 0.6) (layer "F.Cu") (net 8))
 (segment (start 132.799 120.015) (end 133.223 120.439) (width 0.6) (layer "F.Cu") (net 8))
 (segment (start 137.795 106.342) (end 133.985 106.342) (width 0.6) (layer "F.Cu") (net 8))
 (segment (start 130.175 106.68) (end 132.799 106.68) (width 0.6) (layer "F.Cu") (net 8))
 (segment (start 133.053 109.474) (end 133.223 109.304) (width 0.6) (layer "F.Cu") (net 10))
 (segment (start 130.175 122.809) (end 133.053 122.809) (width 0.6) (layer "F.Cu") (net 10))
 (segment (start 133.053 122.809) (end 133.223 122.639) (width 0.6) (layer "F.Cu") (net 10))
 (segment (start 130.175 109.474) (end 133.053 109.474) (width 0.6) (layer "F.Cu") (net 10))
 (segment (start 115.654 115.189) (end 117.305 114.3) (width 0.6) (layer "F.Cu") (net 11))
 (segment (start 117.305 114.3) (end 122.555 114.3) (width 0.6) (layer "F.Cu") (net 11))
 (segment (start 115.654 112.268) (end 115.654 115.189) (width 0.6) (layer "F.Cu") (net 11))
 (segment (start 111.44 104.267) (end 111.76 104.587) (width 0.6) (layer "F.Cu") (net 3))
 (segment (start 110.617 114.681) (end 111.76 113.538) (width 0.6) (layer "F.Cu") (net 3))
 (segment (start 111.76 113.538) (end 111.76 112.268) (width 0.6) (layer "F.Cu") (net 3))
 (segment (start 111.76 110.363) (end 110.744 109.347) (width 0.6) (layer "F.Cu") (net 3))
 (segment (start 110.744 109.347) (end 108.839 109.347) (width 0.6) (layer "F.Cu") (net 3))
 (segment (start 111.76 112.268) (end 111.76 110.363) (width 0.6) (layer "F.Cu") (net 3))
 (segment (start 111.76 104.394) (end 112.268 103.886) (width 0.6) (layer "F.Cu") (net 3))
 (segment (start 112.268 103.886) (end 114.173 103.886) (width 0.6) (layer "F.Cu") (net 3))
 (segment (start 114.173 103.886) (end 114.47 104.183) (width 0.6) (layer "F.Cu") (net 3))
 (segment (start 114.47 104.183) (end 114.47 104.587) (width 0.6) (layer "F.Cu") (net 3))
 (segment (start 107.061 104.267) (end 106.299 105.029) (width 0.6) (layer "F.Cu") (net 3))
 (segment (start 106.299 105.029) (end 106.299 108.458) (width 0.6) (layer "F.Cu") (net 3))
 (segment (start 106.299 108.458) (end 107.188 109.347) (width 0.6) (layer "F.Cu") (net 3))
 (segment (start 107.188 109.347) (end 108.839 109.347) (width 0.6) (layer "F.Cu") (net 3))
 (segment (start 114.239 106.487) (end 111.379 109.347) (width 0.6) (layer "F.Cu") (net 3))
 (segment (start 111.379 109.347) (end 110.744 109.347) (width 0.6) (layer "F.Cu") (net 3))
 (segment (start 108.839 104.267) (end 107.061 104.267) (width 0.6) (layer "F.Cu") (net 3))
 (segment (start 113.454 112.268) (end 111.76 112.268) (width 0.6) (layer "F.Cu") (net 3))
 (segment (start 114.47 106.487) (end 114.239 106.487) (width 0.6) (layer "F.Cu") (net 3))
 (segment (start 111.76 104.587) (end 111.76 104.394) (width 0.6) (layer "F.Cu") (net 3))
 (segment (start 108.839 114.681) (end 110.617 114.681) (width 0.6) (layer "F.Cu") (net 3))
 (segment (start 108.839 104.267) (end 111.44 104.267) (width 0.6) (layer "F.Cu") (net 3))
 (segment (start 112.372 89.027) (end 113.581 90.236) (width 0.6) (layer "F.Cu") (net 13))
 (segment (start 131.93 89.027) (end 133.139 90.236) (width 0.6) (layer "F.Cu") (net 13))
 (segment (start 128.778 89.027) (end 131.93 89.027) (width 0.6) (layer "F.Cu") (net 13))
 (segment (start 109.22 89.027) (end 112.372 89.027) (width 0.6) (layer "F.Cu") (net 13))
 (segment (start 112.776 92.964) (end 108.839 94.107) (width 0.6) (layer "F.Cu") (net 14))
 (segment (start 132.334 92.964) (end 128.397 94.107) (width 0.6) (layer "F.Cu") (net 14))
 (segment (start 133.139 92.136) (end 132.334 92.964) (width 0.6) (layer "F.Cu") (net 14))
 (segment (start 113.581 92.136) (end 112.776 92.964) (width 0.6) (layer "F.Cu") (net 14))
 (segment (start 139.573 104.14) (end 141.224 105.791) (width 0.6) (layer "F.Cu") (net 9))
 (segment (start 130.175 117.475) (end 139.573 117.475) (width 0.6) (layer "F.Cu") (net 9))
 (segment (start 139.573 117.475) (end 141.224 119.126) (width 0.6) (layer "F.Cu") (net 9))
 (segment (start 130.175 104.14) (end 139.573 104.14) (width 0.6) (layer "F.Cu") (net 9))
 (segment (start 137.455 108.882) (end 137.795 108.542) (width 0.6) (layer "F.Cu") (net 12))
 (segment (start 141.013 108.542) (end 141.224 108.331) (width 0.6) (layer "F.Cu") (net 12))
 (segment (start 137.795 121.877) (end 141.013 121.877) (width 0.6) (layer "F.Cu") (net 12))
 (segment (start 141.013 121.877) (end 141.224 121.666) (width 0.6) (layer "F.Cu") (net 12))
 (segment (start 135.636 122.217) (end 137.455 122.217) (width 0.6) (layer "F.Cu") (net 12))
 (segment (start 137.455 122.217) (end 137.795 121.877) (width 0.6) (layer "F.Cu") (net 12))
 (segment (start 135.636 108.882) (end 137.455 108.882) (width 0.6) (layer "F.Cu") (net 12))
 (segment (start 137.795 108.542) (end 141.013 108.542) (width 0.6) (layer "F.Cu") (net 12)))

